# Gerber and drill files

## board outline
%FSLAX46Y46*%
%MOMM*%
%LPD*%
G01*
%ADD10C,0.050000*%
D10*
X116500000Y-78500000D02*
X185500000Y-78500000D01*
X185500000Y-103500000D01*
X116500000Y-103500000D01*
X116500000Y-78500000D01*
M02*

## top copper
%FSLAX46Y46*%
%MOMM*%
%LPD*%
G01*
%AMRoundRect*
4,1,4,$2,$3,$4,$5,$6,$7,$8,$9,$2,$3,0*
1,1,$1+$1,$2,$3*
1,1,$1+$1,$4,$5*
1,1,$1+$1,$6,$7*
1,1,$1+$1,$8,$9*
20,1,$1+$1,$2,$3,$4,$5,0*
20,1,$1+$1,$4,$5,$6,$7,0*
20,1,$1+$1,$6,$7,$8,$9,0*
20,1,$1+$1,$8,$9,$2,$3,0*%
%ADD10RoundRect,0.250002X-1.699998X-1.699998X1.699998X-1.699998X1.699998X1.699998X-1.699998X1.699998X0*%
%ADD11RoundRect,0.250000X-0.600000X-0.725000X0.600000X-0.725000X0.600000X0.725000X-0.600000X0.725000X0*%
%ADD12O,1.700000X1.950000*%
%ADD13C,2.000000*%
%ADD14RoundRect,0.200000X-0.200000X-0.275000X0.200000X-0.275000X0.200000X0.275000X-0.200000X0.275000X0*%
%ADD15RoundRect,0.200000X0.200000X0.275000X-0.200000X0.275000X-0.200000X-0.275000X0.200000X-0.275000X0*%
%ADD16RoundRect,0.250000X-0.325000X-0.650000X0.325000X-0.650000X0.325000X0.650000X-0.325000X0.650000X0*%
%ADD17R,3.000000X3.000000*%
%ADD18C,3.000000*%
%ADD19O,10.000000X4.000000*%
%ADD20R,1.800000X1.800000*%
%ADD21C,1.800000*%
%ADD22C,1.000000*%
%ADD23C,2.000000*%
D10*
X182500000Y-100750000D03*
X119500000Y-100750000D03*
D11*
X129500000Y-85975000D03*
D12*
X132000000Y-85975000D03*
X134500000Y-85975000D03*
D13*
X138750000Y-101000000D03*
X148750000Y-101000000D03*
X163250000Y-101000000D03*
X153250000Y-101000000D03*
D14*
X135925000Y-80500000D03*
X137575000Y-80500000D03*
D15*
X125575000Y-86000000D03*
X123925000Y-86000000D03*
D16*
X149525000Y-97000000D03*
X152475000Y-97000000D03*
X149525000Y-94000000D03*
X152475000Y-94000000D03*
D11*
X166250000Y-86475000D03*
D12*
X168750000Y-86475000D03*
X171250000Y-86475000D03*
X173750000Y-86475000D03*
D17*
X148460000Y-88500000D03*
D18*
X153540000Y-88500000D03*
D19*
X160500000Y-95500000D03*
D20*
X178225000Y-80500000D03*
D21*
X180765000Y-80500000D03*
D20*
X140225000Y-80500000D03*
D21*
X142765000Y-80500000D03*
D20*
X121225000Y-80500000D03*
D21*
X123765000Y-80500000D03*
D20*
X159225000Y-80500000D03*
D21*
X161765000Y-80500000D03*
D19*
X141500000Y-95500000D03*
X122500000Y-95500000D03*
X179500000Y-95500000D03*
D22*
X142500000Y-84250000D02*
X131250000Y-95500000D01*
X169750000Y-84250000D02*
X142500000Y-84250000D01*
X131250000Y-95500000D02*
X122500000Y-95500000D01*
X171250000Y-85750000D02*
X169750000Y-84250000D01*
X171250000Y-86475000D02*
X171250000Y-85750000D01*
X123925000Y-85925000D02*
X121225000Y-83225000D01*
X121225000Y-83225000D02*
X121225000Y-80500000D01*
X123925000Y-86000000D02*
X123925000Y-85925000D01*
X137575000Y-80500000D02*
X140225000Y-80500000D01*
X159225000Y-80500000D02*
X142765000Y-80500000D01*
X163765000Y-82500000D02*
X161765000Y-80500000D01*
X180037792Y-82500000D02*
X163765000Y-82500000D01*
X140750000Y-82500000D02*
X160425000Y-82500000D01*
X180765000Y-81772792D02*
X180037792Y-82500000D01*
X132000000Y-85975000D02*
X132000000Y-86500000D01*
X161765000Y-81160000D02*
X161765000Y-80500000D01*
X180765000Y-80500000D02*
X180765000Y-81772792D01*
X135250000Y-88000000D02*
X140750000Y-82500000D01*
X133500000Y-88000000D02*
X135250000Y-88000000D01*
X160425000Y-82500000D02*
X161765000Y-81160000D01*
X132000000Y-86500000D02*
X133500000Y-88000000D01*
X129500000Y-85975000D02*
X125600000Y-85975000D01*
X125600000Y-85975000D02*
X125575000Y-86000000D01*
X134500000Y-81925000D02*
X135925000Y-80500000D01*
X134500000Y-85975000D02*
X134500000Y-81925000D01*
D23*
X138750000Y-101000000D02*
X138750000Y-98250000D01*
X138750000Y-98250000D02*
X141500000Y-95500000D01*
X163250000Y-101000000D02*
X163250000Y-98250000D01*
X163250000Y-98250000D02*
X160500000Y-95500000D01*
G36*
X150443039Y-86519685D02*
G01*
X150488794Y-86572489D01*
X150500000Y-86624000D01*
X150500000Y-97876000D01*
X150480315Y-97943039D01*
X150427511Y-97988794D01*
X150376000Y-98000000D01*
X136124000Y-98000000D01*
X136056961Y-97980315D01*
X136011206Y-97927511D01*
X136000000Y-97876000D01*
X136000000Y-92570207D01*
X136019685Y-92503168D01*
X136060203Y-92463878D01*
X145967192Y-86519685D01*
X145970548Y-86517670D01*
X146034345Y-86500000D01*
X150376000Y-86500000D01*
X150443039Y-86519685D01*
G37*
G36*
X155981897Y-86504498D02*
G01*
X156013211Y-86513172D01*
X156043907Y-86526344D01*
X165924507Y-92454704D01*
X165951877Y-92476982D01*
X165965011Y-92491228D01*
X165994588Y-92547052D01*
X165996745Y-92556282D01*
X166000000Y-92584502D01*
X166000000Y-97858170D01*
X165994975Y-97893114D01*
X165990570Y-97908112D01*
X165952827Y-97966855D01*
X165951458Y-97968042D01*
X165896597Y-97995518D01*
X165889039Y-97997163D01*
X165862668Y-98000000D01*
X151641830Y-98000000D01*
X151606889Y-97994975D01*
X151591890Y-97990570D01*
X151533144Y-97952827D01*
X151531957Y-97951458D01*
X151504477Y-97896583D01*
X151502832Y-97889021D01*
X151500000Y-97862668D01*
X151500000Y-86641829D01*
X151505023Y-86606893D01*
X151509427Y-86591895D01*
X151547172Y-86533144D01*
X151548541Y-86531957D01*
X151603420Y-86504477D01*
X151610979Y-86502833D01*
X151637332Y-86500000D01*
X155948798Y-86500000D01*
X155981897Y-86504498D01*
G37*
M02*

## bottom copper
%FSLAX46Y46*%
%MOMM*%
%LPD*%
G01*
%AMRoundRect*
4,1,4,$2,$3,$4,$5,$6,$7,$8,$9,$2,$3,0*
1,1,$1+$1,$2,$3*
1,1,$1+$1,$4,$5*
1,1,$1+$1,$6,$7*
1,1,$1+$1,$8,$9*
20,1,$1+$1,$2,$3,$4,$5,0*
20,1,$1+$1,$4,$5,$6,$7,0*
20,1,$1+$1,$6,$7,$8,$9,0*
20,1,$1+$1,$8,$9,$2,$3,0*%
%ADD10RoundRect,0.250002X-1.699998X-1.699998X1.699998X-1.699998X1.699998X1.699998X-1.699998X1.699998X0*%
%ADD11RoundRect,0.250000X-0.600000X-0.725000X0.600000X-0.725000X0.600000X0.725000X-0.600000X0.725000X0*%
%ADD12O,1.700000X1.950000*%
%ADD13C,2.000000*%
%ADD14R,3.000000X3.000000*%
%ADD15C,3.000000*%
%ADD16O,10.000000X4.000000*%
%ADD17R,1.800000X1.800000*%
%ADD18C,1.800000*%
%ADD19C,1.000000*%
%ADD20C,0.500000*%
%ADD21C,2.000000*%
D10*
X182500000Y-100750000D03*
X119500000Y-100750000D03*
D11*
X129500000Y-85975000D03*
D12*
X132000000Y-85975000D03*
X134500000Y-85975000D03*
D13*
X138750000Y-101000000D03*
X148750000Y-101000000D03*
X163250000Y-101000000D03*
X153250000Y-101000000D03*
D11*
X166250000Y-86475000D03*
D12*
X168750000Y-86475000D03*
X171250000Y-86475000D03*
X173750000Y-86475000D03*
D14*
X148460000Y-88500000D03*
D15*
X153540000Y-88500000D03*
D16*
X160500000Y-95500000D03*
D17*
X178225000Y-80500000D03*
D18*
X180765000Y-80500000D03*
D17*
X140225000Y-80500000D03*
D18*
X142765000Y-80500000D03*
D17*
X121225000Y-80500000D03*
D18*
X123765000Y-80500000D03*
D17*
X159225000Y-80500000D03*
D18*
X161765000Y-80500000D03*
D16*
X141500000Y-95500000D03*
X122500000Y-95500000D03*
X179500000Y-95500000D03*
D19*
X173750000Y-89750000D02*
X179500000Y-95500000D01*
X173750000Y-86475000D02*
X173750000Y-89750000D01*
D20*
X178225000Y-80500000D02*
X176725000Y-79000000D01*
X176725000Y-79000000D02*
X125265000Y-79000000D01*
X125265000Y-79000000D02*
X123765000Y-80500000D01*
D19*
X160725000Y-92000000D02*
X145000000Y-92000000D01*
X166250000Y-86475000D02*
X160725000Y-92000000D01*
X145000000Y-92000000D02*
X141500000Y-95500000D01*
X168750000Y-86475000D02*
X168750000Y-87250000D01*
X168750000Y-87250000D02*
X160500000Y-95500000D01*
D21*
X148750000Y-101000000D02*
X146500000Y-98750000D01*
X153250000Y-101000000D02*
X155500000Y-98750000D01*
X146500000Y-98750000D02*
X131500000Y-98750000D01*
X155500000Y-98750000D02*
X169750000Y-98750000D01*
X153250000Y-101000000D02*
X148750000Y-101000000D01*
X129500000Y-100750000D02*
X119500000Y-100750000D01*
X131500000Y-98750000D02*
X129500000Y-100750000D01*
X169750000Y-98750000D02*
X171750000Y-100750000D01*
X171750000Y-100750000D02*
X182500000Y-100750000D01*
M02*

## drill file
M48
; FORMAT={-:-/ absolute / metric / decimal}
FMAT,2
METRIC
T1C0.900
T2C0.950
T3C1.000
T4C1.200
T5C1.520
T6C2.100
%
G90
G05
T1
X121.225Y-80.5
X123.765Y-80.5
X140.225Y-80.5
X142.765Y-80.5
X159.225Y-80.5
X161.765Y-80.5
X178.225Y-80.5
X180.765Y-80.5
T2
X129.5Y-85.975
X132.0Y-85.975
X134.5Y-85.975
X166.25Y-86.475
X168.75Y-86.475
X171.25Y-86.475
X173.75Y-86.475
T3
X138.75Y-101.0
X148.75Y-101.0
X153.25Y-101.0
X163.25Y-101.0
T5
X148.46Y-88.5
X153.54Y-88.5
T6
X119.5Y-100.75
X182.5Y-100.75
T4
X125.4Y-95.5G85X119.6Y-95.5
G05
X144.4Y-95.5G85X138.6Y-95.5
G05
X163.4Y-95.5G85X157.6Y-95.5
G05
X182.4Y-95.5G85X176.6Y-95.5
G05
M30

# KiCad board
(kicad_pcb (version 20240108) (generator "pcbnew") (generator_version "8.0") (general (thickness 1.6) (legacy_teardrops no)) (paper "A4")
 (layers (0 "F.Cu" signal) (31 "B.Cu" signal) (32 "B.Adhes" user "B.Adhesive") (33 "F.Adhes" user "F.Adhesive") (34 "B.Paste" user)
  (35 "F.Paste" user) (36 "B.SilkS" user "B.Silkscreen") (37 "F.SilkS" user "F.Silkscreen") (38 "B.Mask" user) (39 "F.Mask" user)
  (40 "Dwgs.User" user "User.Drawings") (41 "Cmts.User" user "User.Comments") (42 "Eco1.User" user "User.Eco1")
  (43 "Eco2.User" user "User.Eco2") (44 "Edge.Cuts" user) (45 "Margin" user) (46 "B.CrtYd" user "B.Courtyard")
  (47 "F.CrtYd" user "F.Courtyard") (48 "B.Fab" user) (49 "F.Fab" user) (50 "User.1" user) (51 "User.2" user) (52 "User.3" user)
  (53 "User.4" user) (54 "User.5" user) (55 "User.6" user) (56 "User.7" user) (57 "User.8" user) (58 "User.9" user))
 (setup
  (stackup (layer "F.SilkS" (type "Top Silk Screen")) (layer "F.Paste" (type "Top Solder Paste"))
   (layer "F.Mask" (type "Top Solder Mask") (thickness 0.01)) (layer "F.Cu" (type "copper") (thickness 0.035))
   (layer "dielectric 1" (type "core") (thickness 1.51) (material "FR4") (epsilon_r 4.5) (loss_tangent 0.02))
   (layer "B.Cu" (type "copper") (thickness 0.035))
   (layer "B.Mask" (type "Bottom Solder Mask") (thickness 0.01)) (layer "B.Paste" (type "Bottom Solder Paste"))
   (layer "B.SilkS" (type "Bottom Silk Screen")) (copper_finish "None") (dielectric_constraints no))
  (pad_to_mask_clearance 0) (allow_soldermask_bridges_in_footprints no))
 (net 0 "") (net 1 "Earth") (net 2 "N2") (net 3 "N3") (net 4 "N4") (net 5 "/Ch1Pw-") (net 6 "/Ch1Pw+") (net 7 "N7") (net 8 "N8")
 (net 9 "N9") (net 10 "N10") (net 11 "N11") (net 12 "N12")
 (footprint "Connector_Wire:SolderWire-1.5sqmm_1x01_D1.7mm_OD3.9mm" (layer "F.Cu") (at 182.5 100.75)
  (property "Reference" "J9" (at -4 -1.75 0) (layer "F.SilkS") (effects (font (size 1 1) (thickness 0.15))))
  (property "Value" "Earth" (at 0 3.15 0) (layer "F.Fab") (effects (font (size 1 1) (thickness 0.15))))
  (pad "1" thru_hole roundrect (at 0 0) (size 3.9 3.9) (drill 2.1) (layers "*.Cu" "*.Mask") (remove_unused_layers no)
   (roundrect_rratio 0.064103) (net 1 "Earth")))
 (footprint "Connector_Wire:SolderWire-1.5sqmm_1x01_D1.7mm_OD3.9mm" (layer "F.Cu") (at 119.5 100.75)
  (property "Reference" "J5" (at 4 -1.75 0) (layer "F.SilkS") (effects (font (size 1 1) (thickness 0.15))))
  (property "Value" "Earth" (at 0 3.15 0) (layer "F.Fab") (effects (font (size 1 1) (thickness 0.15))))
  (pad "1" thru_hole roundrect (at 0 0) (size 3.9 3.9) (drill 2.1) (layers "*.Cu" "*.Mask") (remove_unused_layers no)
   (roundrect_rratio 0.064103) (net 1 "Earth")))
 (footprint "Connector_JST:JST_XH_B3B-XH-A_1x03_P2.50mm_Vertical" (layer "F.Cu") (at 129.5 85.975)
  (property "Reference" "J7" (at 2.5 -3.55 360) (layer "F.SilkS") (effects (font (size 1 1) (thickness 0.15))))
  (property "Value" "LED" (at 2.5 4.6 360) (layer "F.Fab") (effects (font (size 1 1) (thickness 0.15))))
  (pad "1" thru_hole roundrect (at 0 0) (size 1.7 1.95) (drill 0.95) (layers "*.Cu" "*.Mask") (remove_unused_layers no)
   (roundrect_rratio 0.147059) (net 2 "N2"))
  (pad "2" thru_hole oval (at 2.5 0) (size 1.7 1.95) (drill 0.95) (layers "*.Cu" "*.Mask") (remove_unused_layers no) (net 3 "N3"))
  (pad "3" thru_hole oval (at 5 0) (size 1.7 1.95) (drill 0.95) (layers "*.Cu" "*.Mask") (remove_unused_layers no) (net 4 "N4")))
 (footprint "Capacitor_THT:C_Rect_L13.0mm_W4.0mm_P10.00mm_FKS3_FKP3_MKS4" (layer "F.Cu") (at 138.75 101)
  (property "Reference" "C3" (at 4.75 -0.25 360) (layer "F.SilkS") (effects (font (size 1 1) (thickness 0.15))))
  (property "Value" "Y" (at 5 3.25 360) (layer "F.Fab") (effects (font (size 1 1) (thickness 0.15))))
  (pad "1" thru_hole circle (at 0 0) (size 2 2) (drill 1) (layers "*.Cu" "*.Mask") (remove_unused_layers no) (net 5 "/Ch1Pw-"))
  (pad "2" thru_hole circle (at 10 0) (size 2 2) (drill 1) (layers "*.Cu" "*.Mask") (remove_unused_layers no) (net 1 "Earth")))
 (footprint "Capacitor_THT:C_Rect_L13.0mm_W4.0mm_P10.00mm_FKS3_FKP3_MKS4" (layer "F.Cu") (at 163.25 101 180)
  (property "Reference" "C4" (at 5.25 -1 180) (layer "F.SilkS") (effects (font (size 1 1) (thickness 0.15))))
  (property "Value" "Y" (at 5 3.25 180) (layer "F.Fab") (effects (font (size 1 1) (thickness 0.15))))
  (pad "1" thru_hole circle (at 0 0 180) (size 2 2) (drill 1) (layers "*.Cu" "*.Mask") (remove_unused_layers no) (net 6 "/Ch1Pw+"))
  (pad "2" thru_hole circle (at 10 0 180) (size 2 2) (drill 1) (layers "*.Cu" "*.Mask") (remove_unused_layers no) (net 1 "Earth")))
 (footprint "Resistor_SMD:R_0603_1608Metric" (layer "F.Cu") (at 136.75 80.5)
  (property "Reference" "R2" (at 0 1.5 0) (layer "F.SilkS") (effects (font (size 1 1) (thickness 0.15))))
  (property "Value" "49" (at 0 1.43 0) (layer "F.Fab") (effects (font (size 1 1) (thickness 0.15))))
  (pad "1" smd roundrect (at -0.825 0) (size 0.8 0.95) (layers "F.Cu" "F.Paste" "F.Mask") (roundrect_rratio 0.25) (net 4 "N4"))
  (pad "2" smd roundrect (at 0.825 0) (size 0.8 0.95) (layers "F.Cu" "F.Paste" "F.Mask") (roundrect_rratio 0.25) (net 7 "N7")))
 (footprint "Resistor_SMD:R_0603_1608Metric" (layer "F.Cu") (at 124.75 86 180)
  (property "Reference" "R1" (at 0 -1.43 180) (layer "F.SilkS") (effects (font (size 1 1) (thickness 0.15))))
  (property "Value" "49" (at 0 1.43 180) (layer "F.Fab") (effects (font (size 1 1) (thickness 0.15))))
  (pad "1" smd roundrect (at -0.825 0 180) (size 0.8 0.95) (layers "F.Cu" "F.Paste" "F.Mask") (roundrect_rratio 0.25) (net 2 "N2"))
  (pad "2" smd roundrect (at 0.825 0 180) (size 0.8 0.95) (layers "F.Cu" "F.Paste" "F.Mask") (roundrect_rratio 0.25) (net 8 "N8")))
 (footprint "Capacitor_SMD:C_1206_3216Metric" (layer "F.Cu") (at 151 97)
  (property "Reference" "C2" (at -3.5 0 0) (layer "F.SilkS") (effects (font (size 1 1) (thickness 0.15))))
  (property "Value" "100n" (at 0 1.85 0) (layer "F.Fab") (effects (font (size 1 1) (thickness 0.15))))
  (pad "1" smd roundrect (at -1.475 0) (size 1.15 1.8) (layers "F.Cu" "F.Paste" "F.Mask") (roundrect_rratio 0.217391) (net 5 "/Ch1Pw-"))
  (pad "2" smd roundrect (at 1.475 0) (size 1.15 1.8) (layers "F.Cu" "F.Paste" "F.Mask") (roundrect_rratio 0.217391) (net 6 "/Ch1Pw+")))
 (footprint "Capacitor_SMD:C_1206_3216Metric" (layer "F.Cu") (at 151 94)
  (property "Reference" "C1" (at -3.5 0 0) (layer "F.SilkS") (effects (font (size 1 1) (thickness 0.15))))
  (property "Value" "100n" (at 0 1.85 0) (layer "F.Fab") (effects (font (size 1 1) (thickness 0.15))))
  (pad "1" smd roundrect (at -1.475 0) (size 1.15 1.8) (layers "F.Cu" "F.Paste" "F.Mask") (roundrect_rratio 0.217391) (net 5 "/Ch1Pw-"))
  (pad "2" smd roundrect (at 1.475 0) (size 1.15 1.8) (layers "F.Cu" "F.Paste" "F.Mask") (roundrect_rratio 0.217391) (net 6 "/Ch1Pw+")))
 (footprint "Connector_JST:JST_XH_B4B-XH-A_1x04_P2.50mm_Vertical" (layer "F.Cu") (at 166.25 86.475)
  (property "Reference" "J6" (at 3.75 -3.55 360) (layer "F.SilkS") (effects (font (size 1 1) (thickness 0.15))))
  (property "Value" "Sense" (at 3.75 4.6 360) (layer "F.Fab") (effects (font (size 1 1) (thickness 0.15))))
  (pad "1" thru_hole roundrect (at 0 0) (size 1.7 1.95) (drill 0.95) (layers "*.Cu" "*.Mask") (remove_unused_layers no)
   (roundrect_rratio 0.147059) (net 5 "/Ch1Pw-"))
  (pad "2" thru_hole oval (at 2.5 0) (size 1.7 1.95) (drill 0.95) (layers "*.Cu" "*.Mask") (remove_unused_layers no) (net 6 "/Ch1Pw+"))
  (pad "3" thru_hole oval (at 5 0) (size 1.7 1.95) (drill 0.95) (layers "*.Cu" "*.Mask") (remove_unused_layers no) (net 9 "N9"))
  (pad "4" thru_hole oval (at 7.5 0) (size 1.7 1.95) (drill 0.95) (layers "*.Cu" "*.Mask") (remove_unused_layers no) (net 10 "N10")))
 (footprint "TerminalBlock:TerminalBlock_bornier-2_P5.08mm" (layer "F.Cu") (at 148.46 88.5)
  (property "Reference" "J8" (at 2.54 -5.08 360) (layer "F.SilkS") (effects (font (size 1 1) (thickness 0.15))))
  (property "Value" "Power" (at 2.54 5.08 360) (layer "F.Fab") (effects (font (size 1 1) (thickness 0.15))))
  (pad "1" thru_hole rect (at 0 0) (size 3 3) (drill 1.52) (layers "*.Cu" "*.Mask") (remove_unused_layers no) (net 5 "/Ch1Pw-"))
  (pad "2" thru_hole circle (at 5.08 0) (size 3 3) (drill 1.52) (layers "*.Cu" "*.Mask") (remove_unused_layers no) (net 6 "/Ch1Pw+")))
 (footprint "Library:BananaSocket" (layer "B.Cu") (at 160.5 95.5 180)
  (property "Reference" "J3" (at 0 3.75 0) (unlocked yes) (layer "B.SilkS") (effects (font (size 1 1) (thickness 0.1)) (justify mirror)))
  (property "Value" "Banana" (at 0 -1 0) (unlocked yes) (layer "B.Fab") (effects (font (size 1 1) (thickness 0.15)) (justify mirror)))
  (pad "1" thru_hole oval (at 0 0 180) (size 10 4) (drill oval 7 1.2) (layers "*.Cu" "*.Mask") (remove_unused_layers no) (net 6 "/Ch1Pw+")))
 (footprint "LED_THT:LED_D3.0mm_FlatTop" (layer "B.Cu") (at 178.225 80.5)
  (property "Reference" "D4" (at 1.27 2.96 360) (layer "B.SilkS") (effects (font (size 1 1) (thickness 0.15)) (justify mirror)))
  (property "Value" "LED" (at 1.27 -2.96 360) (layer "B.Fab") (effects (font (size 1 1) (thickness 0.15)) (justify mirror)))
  (pad "1" thru_hole rect (at 0 0) (size 1.8 1.8) (drill 0.9) (layers "*.Cu" "*.Mask") (remove_unused_layers no) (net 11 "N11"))
  (pad "2" thru_hole circle (at 2.54 0) (size 1.8 1.8) (drill 0.9) (layers "*.Cu" "*.Mask") (remove_unused_layers no) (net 3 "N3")))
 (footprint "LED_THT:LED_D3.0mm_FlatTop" (layer "B.Cu") (at 140.225 80.5)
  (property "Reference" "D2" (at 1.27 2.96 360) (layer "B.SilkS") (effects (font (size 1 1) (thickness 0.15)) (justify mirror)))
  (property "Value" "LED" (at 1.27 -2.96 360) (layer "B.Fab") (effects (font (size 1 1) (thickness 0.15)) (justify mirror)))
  (pad "1" thru_hole rect (at 0 0) (size 1.8 1.8) (drill 0.9) (layers "*.Cu" "*.Mask") (remove_unused_layers no) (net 7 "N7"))
  (pad "2" thru_hole circle (at 2.54 0) (size 1.8 1.8) (drill 0.9) (layers "*.Cu" "*.Mask") (remove_unused_layers no) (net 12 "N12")))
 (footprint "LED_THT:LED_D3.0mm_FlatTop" (layer "B.Cu") (at 121.225 80.5)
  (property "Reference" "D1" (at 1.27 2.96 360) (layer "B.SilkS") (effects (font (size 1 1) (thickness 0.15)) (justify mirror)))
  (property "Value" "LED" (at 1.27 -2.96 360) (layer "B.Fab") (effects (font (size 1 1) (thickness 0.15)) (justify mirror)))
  (pad "1" thru_hole rect (at 0 0) (size 1.8 1.8) (drill 0.9) (layers "*.Cu" "*.Mask") (remove_unused_layers no) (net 8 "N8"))
  (pad "2" thru_hole circle (at 2.54 0) (size 1.8 1.8) (drill 0.9) (layers "*.Cu" "*.Mask") (remove_unused_layers no) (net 11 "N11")))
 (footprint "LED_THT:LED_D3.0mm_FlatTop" (layer "B.Cu") (at 159.225 80.5)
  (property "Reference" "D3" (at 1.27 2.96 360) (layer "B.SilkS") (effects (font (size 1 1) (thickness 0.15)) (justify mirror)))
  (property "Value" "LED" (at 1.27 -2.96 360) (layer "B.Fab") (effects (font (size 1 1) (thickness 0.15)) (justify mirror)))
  (pad "1" thru_hole rect (at 0 0) (size 1.8 1.8) (drill 0.9) (layers "*.Cu" "*.Mask") (remove_unused_layers no) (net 12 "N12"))
  (pad "2" thru_hole circle (at 2.54 0) (size 1.8 1.8) (drill 0.9) (layers "*.Cu" "*.Mask") (remove_unused_layers no) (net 3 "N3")))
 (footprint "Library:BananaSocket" (layer "B.Cu") (at 141.5 95.5 180)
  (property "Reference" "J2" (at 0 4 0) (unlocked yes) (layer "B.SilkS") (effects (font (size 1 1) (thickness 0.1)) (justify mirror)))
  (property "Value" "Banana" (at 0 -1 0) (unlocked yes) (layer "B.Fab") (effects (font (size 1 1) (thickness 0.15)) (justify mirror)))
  (pad "1" thru_hole oval (at 0 0 180) (size 10 4) (drill oval 7 1.2) (layers "*.Cu" "*.Mask") (remove_unused_layers no) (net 5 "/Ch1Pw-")))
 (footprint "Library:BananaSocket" (layer "B.Cu") (at 122.5 95.5 180)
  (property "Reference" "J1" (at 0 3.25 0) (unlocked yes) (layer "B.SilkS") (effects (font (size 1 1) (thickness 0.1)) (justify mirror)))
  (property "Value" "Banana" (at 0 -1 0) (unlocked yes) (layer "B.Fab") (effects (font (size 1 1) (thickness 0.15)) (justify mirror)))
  (pad "1" thru_hole oval (at 0 0 180) (size 10 4) (drill oval 7 1.2) (layers "*.Cu" "*.Mask") (remove_unused_layers no) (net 9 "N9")))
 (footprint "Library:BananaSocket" (layer "B.Cu") (at 179.5 95.5 180)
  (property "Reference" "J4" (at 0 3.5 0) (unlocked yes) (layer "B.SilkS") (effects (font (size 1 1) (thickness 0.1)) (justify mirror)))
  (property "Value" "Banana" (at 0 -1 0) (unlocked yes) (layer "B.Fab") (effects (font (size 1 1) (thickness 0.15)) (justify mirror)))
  (pad "1" thru_hole oval (at 0 0 180) (size 10 4) (drill oval 7 1.2) (layers "*.Cu" "*.Mask") (remove_unused_layers no) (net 10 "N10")))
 (gr_rect (start 116.5 78.5) (end 185.5 103.5) (stroke (width 0.05) (type default)) (fill none) (layer "Edge.Cuts"))
 (segment (start 142.5 84.25) (end 131.25 95.5) (width 1) (layer "F.Cu") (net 9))
 (segment (start 169.75 84.25) (end 142.5 84.25) (width 1) (layer "F.Cu") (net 9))
 (segment (start 131.25 95.5) (end 122.5 95.5) (width 1) (layer "F.Cu") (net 9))
 (segment (start 171.25 85.75) (end 169.75 84.25) (width 1) (layer "F.Cu") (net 9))
 (segment (start 171.25 86.475) (end 171.25 85.75) (width 1) (layer "F.Cu") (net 9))
 (segment (start 173.75 89.75) (end 179.5 95.5) (width 1) (layer "B.Cu") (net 10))
 (segment (start 173.75 86.475) (end 173.75 89.75) (width 1) (layer "B.Cu") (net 10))
 (segment (start 178.225 80.5) (end 176.725 79) (width 0.5) (layer "B.Cu") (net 11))
 (segment (start 176.725 79) (end 125.265 79) (width 0.5) (layer "B.Cu") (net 11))
 (segment (start 125.265 79) (end 123.765 80.5) (width 0.5) (layer "B.Cu") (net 11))
 (segment (start 123.925 85.925) (end 121.225 83.225) (width 1) (layer "F.Cu") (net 8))
 (segment (start 121.225 83.225) (end 121.225 80.5) (width 1) (layer "F.Cu") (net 8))
 (segment (start 123.925 86) (end 123.925 85.925) (width 1) (layer "F.Cu") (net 8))
 (segment (start 137.575 80.5) (end 140.225 80.5) (width 1) (layer "F.Cu") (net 7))
 (segment (start 159.225 80.5) (end 142.765 80.5) (width 1) (layer "F.Cu") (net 12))
 (segment (start 163.765 82.5) (end 161.765 80.5) (width 1) (layer "F.Cu") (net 3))
 (segment (start 180.037792 82.5) (end 163.765 82.5) (width 1) (layer "F.Cu") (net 3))
 (segment (start 140.75 82.5) (end 160.425 82.5) (width 1) (layer "F.Cu") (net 3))
 (segment (start 180.765 81.772792) (end 180.037792 82.5) (width 1) (layer "F.Cu") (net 3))
 (segment (start 132 85.975) (end 132 86.5) (width 1) (layer "F.Cu") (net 3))
 (segment (start 161.765 81.16) (end 161.765 80.5) (width 1) (layer "F.Cu") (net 3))
 (segment (start 180.765 80.5) (end 180.765 81.772792) (width 1) (layer "F.Cu") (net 3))
 (segment (start 135.25 88) (end 140.75 82.5) (width 1) (layer "F.Cu") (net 3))
 (segment (start 133.5 88) (end 135.25 88) (width 1) (layer "F.Cu") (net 3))
 (segment (start 160.425 82.5) (end 161.765 81.16) (width 1) (layer "F.Cu") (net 3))
 (segment (start 132 86.5) (end 133.5 88) (width 1) (layer "F.Cu") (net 3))
 (segment (start 129.5 85.975) (end 125.6 85.975) (width 1) (layer "F.Cu") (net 2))
 (segment (start 125.6 85.975) (end 125.575 86) (width 1) (layer "F.Cu") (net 2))
 (segment (start 134.5 81.925) (end 135.925 80.5) (width 1) (layer "F.Cu") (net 4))
 (segment (start 134.5 85.975) (end 134.5 81.925) (width 1) (layer "F.Cu") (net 4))
 (segment (start 138.75 101) (end 138.75 98.25) (width 2) (layer "F.Cu") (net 5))
 (segment (start 138.75 98.25) (end 141.5 95.5) (width 2) (layer "F.Cu") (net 5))
 (segment (start 160.725 92) (end 145 92) (width 1) (layer "B.Cu") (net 5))
 (segment (start 166.25 86.475) (end 160.725 92) (width 1) (layer "B.Cu") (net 5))
 (segment (start 145 92) (end 141.5 95.5) (width 1) (layer "B.Cu") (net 5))
 (segment (start 163.25 101) (end 163.25 98.25) (width 2) (layer "F.Cu") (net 6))
 (segment (start 163.25 98.25) (end 160.5 95.5) (width 2) (layer "F.Cu") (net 6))
 (segment (start 168.75 86.475) (end 168.75 87.25) (width 1) (layer "B.Cu") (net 6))
 (segment (start 168.75 87.25) (end 160.5 95.5) (width 1) (layer "B.Cu") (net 6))
 (segment (start 148.75 101) (end 146.5 98.75) (width 2) (layer "B.Cu") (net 1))
 (segment (start 153.25 101) (end 155.5 98.75) (width 2) (layer "B.Cu") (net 1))
 (segment (start 146.5 98.75) (end 131.5 98.75) (width 2) (layer "B.Cu") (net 1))
 (segment (start 155.5 98.75) (end 169.75 98.75) (width 2) (layer "B.Cu") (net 1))
 (segment (start 153.25 101) (end 148.75 101) (width 2) (layer "B.Cu") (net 1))
 (segment (start 129.5 100.75) (end 119.5 100.75) (width 2) (layer "B.Cu") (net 1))
 (segment (start 131.5 98.75) (end 129.5 100.75) (width 2) (layer "B.Cu") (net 1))
 (segment (start 169.75 98.75) (end 171.75 100.75) (width 2) (layer "B.Cu") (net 1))
 (segment (start 171.75 100.75) (end 182.5 100.75) (width 2) (layer "B.Cu") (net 1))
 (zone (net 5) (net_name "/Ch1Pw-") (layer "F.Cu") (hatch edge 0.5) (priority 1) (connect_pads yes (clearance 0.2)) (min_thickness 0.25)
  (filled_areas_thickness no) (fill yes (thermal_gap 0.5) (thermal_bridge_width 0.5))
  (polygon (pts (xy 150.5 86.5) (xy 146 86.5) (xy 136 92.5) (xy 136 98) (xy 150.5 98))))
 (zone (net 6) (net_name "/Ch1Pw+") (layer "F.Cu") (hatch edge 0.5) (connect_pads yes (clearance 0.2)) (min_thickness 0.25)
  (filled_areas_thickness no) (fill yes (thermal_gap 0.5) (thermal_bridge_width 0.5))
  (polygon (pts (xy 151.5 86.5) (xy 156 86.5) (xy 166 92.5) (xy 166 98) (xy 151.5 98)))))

